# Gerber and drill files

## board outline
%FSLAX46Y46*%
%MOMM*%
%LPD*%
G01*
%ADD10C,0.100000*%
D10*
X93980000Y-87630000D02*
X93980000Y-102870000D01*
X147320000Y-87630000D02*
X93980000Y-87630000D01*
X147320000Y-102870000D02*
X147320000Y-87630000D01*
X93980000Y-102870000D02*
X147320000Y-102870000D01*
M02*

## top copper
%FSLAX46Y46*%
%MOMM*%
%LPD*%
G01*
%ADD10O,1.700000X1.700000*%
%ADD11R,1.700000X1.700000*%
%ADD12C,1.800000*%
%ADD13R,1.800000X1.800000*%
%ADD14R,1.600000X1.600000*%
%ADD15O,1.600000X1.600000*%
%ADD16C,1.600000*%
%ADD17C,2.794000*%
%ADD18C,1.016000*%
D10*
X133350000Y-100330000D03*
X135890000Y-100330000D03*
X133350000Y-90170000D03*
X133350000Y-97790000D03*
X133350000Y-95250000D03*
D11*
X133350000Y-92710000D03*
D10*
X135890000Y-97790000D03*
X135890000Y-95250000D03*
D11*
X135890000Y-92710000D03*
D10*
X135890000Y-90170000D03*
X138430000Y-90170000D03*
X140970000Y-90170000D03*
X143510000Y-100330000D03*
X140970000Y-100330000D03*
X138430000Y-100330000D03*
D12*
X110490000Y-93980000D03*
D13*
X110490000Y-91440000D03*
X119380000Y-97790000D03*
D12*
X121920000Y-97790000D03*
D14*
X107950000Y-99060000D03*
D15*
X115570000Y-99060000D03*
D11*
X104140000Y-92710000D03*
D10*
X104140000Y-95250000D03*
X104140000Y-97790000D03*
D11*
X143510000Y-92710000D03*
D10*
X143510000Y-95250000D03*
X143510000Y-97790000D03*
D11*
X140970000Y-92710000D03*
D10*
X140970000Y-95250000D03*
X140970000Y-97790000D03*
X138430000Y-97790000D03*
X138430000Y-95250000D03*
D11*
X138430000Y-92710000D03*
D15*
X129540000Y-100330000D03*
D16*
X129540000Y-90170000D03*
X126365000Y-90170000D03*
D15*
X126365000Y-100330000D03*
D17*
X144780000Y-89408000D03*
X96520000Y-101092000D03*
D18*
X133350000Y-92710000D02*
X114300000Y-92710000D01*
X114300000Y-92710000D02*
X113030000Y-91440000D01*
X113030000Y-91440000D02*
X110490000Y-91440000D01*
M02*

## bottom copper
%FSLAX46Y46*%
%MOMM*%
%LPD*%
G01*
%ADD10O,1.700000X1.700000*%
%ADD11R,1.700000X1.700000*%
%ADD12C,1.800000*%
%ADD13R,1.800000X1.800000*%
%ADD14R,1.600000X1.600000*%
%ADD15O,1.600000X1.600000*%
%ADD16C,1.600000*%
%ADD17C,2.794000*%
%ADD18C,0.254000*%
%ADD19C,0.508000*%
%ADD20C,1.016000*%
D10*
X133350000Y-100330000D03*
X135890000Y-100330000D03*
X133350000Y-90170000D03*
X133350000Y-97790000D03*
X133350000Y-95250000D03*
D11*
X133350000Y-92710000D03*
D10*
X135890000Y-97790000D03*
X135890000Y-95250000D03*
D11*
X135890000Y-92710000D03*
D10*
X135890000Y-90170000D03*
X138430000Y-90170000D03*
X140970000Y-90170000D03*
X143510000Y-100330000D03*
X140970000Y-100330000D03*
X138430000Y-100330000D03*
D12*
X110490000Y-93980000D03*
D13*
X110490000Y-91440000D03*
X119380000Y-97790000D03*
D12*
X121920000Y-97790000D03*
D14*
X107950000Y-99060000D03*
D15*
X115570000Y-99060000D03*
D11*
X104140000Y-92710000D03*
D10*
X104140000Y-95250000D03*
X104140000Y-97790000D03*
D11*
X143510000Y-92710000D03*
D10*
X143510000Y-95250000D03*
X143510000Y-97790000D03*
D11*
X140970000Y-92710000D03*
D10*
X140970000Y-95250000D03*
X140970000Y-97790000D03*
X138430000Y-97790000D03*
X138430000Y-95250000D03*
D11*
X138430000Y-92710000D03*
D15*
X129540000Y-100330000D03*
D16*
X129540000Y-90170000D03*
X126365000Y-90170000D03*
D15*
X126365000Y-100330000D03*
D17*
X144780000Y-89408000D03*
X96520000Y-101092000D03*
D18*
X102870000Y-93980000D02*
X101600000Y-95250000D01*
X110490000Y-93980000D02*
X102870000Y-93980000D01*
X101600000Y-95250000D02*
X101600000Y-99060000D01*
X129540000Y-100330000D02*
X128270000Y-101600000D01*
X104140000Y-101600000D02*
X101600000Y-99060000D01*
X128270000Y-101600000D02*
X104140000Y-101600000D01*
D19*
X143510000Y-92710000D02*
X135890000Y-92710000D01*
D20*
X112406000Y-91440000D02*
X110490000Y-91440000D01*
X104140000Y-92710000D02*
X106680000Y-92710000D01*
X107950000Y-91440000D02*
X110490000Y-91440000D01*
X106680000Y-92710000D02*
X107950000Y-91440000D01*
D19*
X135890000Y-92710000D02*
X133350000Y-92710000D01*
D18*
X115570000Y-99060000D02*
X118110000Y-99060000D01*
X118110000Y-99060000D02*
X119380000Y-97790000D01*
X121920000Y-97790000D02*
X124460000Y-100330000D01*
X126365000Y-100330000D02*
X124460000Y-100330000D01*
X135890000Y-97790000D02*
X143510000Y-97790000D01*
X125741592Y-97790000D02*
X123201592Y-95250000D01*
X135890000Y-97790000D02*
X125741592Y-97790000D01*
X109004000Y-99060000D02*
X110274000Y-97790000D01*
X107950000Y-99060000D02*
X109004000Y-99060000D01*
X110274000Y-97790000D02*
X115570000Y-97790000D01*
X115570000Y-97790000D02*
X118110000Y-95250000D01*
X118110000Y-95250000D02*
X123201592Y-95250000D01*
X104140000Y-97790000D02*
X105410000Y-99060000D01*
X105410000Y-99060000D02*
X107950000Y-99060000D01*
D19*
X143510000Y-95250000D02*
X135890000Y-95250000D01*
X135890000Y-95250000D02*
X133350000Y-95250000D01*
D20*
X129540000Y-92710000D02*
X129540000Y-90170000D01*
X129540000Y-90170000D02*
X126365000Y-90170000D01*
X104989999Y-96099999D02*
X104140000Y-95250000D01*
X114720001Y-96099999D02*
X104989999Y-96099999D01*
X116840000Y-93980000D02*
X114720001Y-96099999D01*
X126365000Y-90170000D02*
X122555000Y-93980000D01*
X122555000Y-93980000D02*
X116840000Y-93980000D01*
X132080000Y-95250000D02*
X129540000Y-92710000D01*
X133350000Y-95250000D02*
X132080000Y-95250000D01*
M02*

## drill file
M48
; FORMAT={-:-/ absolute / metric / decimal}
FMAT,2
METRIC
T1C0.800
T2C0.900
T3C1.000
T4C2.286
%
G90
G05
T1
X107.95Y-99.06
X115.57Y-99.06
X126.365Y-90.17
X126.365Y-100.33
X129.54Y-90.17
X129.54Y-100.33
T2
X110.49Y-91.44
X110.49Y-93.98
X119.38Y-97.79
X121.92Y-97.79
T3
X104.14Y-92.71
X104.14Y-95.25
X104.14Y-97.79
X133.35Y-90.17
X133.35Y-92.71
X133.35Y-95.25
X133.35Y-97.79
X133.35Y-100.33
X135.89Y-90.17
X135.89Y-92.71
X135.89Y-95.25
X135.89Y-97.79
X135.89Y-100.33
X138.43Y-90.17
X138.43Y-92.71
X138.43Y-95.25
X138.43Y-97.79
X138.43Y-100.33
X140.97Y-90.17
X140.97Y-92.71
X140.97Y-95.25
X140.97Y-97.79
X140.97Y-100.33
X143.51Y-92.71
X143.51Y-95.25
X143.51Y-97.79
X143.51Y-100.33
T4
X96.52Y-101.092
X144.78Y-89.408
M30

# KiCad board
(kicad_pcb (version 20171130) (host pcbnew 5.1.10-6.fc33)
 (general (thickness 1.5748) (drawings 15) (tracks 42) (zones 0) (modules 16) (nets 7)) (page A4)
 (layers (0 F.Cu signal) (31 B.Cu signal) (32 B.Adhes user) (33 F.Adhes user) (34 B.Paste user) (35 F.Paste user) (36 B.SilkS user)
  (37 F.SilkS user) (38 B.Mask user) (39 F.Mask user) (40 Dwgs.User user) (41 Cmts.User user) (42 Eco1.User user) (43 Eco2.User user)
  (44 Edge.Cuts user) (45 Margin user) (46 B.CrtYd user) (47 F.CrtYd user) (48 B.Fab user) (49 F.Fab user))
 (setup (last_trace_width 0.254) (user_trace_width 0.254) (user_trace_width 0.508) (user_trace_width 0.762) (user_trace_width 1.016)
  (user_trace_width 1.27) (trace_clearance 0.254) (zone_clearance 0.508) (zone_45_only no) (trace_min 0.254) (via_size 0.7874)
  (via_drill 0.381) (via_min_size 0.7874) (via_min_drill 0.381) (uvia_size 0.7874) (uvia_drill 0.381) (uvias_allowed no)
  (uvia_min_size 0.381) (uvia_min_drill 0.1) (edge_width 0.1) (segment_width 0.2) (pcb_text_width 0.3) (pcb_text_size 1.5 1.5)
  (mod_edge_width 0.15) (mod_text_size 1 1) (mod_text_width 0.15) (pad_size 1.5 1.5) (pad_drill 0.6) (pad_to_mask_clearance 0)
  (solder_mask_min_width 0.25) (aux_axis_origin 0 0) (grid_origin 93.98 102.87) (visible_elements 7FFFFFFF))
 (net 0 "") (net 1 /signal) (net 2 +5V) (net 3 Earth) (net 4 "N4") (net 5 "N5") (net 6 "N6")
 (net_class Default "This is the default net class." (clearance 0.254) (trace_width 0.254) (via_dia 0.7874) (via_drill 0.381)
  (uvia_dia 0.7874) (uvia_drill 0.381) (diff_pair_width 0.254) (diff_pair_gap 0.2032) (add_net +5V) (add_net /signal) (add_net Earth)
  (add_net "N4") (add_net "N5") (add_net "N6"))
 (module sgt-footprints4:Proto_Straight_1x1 (layer F.Cu) (at 133.35 100.33)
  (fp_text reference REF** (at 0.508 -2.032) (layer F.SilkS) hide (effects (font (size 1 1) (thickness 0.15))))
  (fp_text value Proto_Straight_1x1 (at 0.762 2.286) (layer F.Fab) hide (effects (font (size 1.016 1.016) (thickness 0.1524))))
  (pad 1 thru_hole oval (at 0 0) (size 1.7 1.7) (drill 1) (layers *.Cu *.Mask)))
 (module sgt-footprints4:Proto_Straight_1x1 (layer F.Cu) (at 135.89 100.33)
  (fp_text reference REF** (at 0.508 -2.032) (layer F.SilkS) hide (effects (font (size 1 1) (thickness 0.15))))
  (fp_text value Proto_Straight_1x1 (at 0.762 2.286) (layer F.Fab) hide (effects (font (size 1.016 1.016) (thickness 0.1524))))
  (pad 1 thru_hole oval (at 0 0) (size 1.7 1.7) (drill 1) (layers *.Cu *.Mask)))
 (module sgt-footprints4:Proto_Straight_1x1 (layer F.Cu) (at 133.35 90.17)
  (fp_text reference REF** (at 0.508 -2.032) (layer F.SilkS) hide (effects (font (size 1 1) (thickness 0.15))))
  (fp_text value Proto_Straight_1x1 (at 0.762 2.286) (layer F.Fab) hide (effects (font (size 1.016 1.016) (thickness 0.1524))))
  (pad 1 thru_hole oval (at 0 0) (size 1.7 1.7) (drill 1) (layers *.Cu *.Mask)))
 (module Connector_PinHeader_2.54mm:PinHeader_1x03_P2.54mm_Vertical (layer F.Cu) (at 133.35 92.71)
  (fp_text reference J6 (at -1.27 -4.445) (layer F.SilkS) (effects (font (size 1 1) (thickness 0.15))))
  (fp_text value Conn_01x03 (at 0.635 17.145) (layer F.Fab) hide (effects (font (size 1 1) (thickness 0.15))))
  (pad 3 thru_hole oval (at 0 5.08) (size 1.7 1.7) (drill 1) (layers *.Cu *.Mask) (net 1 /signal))
  (pad 2 thru_hole oval (at 0 2.54) (size 1.7 1.7) (drill 1) (layers *.Cu *.Mask) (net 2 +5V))
  (pad 1 thru_hole rect (at 0 0) (size 1.7 1.7) (drill 1) (layers *.Cu *.Mask) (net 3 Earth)))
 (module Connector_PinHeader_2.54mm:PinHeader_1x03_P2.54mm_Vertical (layer F.Cu) (at 135.89 92.71)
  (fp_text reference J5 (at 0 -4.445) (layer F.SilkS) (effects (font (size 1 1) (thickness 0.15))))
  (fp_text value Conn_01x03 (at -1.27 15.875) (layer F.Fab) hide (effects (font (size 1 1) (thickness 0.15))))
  (pad 3 thru_hole oval (at 0 5.08) (size 1.7 1.7) (drill 1) (layers *.Cu *.Mask) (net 1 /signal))
  (pad 2 thru_hole oval (at 0 2.54) (size 1.7 1.7) (drill 1) (layers *.Cu *.Mask) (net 2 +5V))
  (pad 1 thru_hole rect (at 0 0) (size 1.7 1.7) (drill 1) (layers *.Cu *.Mask) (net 3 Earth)))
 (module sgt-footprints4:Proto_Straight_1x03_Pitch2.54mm (layer F.Cu) (at 135.89 90.17 90)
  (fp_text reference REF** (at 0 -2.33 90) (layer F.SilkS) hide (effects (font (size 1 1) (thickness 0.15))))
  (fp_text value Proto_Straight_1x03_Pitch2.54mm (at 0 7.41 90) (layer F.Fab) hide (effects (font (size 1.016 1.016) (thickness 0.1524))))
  (pad 1 thru_hole oval (at 0 0 90) (size 1.7 1.7) (drill 1) (layers *.Cu *.Mask))
  (pad 2 thru_hole oval (at 0 2.54 90) (size 1.7 1.7) (drill 1) (layers *.Cu *.Mask))
  (pad 3 thru_hole oval (at 0 5.08 90) (size 1.7 1.7) (drill 1) (layers *.Cu *.Mask)))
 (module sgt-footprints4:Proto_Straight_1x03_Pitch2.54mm (layer F.Cu) (at 138.43 100.33 90)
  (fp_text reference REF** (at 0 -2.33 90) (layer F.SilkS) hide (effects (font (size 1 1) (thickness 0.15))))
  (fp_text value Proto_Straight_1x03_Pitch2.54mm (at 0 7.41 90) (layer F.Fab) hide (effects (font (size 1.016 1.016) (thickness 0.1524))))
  (pad 3 thru_hole oval (at 0 5.08 90) (size 1.7 1.7) (drill 1) (layers *.Cu *.Mask))
  (pad 2 thru_hole oval (at 0 2.54 90) (size 1.7 1.7) (drill 1) (layers *.Cu *.Mask))
  (pad 1 thru_hole oval (at 0 0 90) (size 1.7 1.7) (drill 1) (layers *.Cu *.Mask)))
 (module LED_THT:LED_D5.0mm (layer F.Cu) (at 110.49 91.44 270)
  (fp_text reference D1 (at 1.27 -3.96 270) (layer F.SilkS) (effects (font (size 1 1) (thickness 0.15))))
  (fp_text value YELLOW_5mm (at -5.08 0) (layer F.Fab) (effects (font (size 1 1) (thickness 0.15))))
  (pad 2 thru_hole circle (at 2.54 0 270) (size 1.8 1.8) (drill 0.9) (layers *.Cu *.Mask) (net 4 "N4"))
  (pad 1 thru_hole rect (at 0 0 270) (size 1.8 1.8) (drill 0.9) (layers *.Cu *.Mask) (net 3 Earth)))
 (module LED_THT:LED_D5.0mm (layer F.Cu) (at 119.38 97.79)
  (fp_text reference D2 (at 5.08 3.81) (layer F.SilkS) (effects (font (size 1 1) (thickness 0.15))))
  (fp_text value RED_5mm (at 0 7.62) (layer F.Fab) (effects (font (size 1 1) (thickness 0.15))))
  (pad 1 thru_hole rect (at 0 0) (size 1.8 1.8) (drill 0.9) (layers *.Cu *.Mask) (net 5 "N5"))
  (pad 2 thru_hole circle (at 2.54 0) (size 1.8 1.8) (drill 0.9) (layers *.Cu *.Mask) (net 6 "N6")))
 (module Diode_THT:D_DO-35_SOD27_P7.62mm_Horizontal (layer F.Cu) (at 107.95 99.06)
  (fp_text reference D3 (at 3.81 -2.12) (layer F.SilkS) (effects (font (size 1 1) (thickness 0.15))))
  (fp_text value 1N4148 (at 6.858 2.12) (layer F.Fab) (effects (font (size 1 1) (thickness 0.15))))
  (pad 1 thru_hole rect (at 0 0) (size 1.6 1.6) (drill 0.8) (layers *.Cu *.Mask) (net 1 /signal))
  (pad 2 thru_hole oval (at 7.62 0) (size 1.6 1.6) (drill 0.8) (layers *.Cu *.Mask) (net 5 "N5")))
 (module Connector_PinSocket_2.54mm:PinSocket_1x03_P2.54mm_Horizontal (layer F.Cu) (at 104.14 92.71)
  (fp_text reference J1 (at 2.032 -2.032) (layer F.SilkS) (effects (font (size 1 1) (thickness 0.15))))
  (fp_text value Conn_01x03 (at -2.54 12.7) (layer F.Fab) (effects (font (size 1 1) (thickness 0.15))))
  (pad 1 thru_hole rect (at 0 0) (size 1.7 1.7) (drill 1) (layers *.Cu *.Mask) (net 3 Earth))
  (pad 2 thru_hole oval (at 0 2.54) (size 1.7 1.7) (drill 1) (layers *.Cu *.Mask) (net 2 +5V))
  (pad 3 thru_hole oval (at 0 5.08) (size 1.7 1.7) (drill 1) (layers *.Cu *.Mask) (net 1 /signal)))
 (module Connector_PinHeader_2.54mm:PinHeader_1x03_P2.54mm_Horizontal (layer F.Cu) (at 143.51 92.71)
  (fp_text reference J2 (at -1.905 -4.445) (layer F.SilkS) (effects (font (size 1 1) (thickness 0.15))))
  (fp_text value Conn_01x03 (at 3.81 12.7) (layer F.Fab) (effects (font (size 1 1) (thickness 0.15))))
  (pad 1 thru_hole rect (at 0 0) (size 1.7 1.7) (drill 1) (layers *.Cu *.Mask) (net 3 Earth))
  (pad 2 thru_hole oval (at 0 2.54) (size 1.7 1.7) (drill 1) (layers *.Cu *.Mask) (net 2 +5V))
  (pad 3 thru_hole oval (at 0 5.08) (size 1.7 1.7) (drill 1) (layers *.Cu *.Mask) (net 1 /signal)))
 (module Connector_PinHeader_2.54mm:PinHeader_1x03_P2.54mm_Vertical (layer F.Cu) (at 140.97 92.71)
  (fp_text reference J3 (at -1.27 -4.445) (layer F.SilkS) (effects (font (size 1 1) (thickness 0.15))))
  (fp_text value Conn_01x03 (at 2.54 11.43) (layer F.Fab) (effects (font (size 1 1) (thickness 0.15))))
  (pad 1 thru_hole rect (at 0 0) (size 1.7 1.7) (drill 1) (layers *.Cu *.Mask) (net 3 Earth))
  (pad 2 thru_hole oval (at 0 2.54) (size 1.7 1.7) (drill 1) (layers *.Cu *.Mask) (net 2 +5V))
  (pad 3 thru_hole oval (at 0 5.08) (size 1.7 1.7) (drill 1) (layers *.Cu *.Mask) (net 1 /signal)))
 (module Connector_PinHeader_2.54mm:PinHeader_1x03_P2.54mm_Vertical (layer F.Cu) (at 138.43 92.71)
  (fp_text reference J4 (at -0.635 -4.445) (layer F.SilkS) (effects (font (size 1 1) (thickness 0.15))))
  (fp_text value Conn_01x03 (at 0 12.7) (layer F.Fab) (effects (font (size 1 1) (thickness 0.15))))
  (pad 3 thru_hole oval (at 0 5.08) (size 1.7 1.7) (drill 1) (layers *.Cu *.Mask) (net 1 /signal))
  (pad 2 thru_hole oval (at 0 2.54) (size 1.7 1.7) (drill 1) (layers *.Cu *.Mask) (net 2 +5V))
  (pad 1 thru_hole rect (at 0 0) (size 1.7 1.7) (drill 1) (layers *.Cu *.Mask) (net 3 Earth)))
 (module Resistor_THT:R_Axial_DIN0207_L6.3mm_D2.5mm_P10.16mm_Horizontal (layer F.Cu) (at 129.54 90.17 270)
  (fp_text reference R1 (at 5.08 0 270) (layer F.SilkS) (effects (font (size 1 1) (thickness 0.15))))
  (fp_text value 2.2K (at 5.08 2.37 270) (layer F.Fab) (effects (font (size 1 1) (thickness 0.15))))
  (pad 2 thru_hole oval (at 10.16 0 270) (size 1.6 1.6) (drill 0.8) (layers *.Cu *.Mask) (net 4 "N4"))
  (pad 1 thru_hole circle (at 0 0 270) (size 1.6 1.6) (drill 0.8) (layers *.Cu *.Mask) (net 2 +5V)))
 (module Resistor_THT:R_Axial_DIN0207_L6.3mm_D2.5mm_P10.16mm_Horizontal (layer F.Cu) (at 126.365 90.17 270)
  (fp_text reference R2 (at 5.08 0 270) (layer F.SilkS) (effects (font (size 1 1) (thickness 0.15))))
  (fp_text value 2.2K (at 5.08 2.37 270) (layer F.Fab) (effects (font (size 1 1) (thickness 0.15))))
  (pad 1 thru_hole circle (at 0 0 270) (size 1.6 1.6) (drill 0.8) (layers *.Cu *.Mask) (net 2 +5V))
  (pad 2 thru_hole oval (at 10.16 0 270) (size 1.6 1.6) (drill 0.8) (layers *.Cu *.Mask) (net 6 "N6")))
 (gr_line (start 93.98 87.63) (end 93.98 102.87) (layer Edge.Cuts) (width 0.1))
 (gr_line (start 147.32 87.63) (end 93.98 87.63) (layer Edge.Cuts) (width 0.1))
 (gr_line (start 147.32 102.87) (end 147.32 87.63) (layer Edge.Cuts) (width 0.1))
 (gr_line (start 93.98 102.87) (end 147.32 102.87) (layer Edge.Cuts) (width 0.1))
 (via (at 144.78 89.408) (size 2.794) (drill 2.286) (layers F.Cu B.Cu) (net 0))
 (via (at 96.52 101.092) (size 2.794) (drill 2.286) (layers F.Cu B.Cu) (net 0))
 (segment (start 102.87 93.98) (end 101.6 95.25) (width 0.254) (layer B.Cu) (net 4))
 (segment (start 110.49 93.98) (end 102.87 93.98) (width 0.254) (layer B.Cu) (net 4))
 (segment (start 101.6 95.25) (end 101.6 99.06) (width 0.254) (layer B.Cu) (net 4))
 (segment (start 129.54 100.33) (end 128.27 101.6) (width 0.254) (layer B.Cu) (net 4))
 (segment (start 104.14 101.6) (end 101.6 99.06) (width 0.254) (layer B.Cu) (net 4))
 (segment (start 128.27 101.6) (end 104.14 101.6) (width 0.254) (layer B.Cu) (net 4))
 (segment (start 143.51 92.71) (end 135.89 92.71) (width 0.508) (layer B.Cu) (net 3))
 (segment (start 112.406 91.44) (end 110.49 91.44) (width 1.016) (layer B.Cu) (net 3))
 (segment (start 104.14 92.71) (end 106.68 92.71) (width 1.016) (layer B.Cu) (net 3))
 (segment (start 107.95 91.44) (end 110.49 91.44) (width 1.016) (layer B.Cu) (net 3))
 (segment (start 106.68 92.71) (end 107.95 91.44) (width 1.016) (layer B.Cu) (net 3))
 (segment (start 135.89 92.71) (end 133.35 92.71) (width 0.508) (layer B.Cu) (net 3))
 (segment (start 133.35 92.71) (end 114.3 92.71) (width 1.016) (layer F.Cu) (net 3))
 (segment (start 114.3 92.71) (end 113.03 91.44) (width 1.016) (layer F.Cu) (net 3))
 (segment (start 113.03 91.44) (end 110.49 91.44) (width 1.016) (layer F.Cu) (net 3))
 (segment (start 115.57 99.06) (end 118.11 99.06) (width 0.254) (layer B.Cu) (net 5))
 (segment (start 118.11 99.06) (end 119.38 97.79) (width 0.254) (layer B.Cu) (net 5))
 (segment (start 121.92 97.79) (end 124.46 100.33) (width 0.254) (layer B.Cu) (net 6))
 (segment (start 126.365 100.33) (end 124.46 100.33) (width 0.254) (layer B.Cu) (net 6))
 (segment (start 135.89 97.79) (end 143.51 97.79) (width 0.254) (layer B.Cu) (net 1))
 (segment (start 125.741592 97.79) (end 123.201592 95.25) (width 0.254) (layer B.Cu) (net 1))
 (segment (start 135.89 97.79) (end 125.741592 97.79) (width 0.254) (layer B.Cu) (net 1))
 (segment (start 109.004 99.06) (end 110.274 97.79) (width 0.254) (layer B.Cu) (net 1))
 (segment (start 107.95 99.06) (end 109.004 99.06) (width 0.254) (layer B.Cu) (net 1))
 (segment (start 110.274 97.79) (end 115.57 97.79) (width 0.254) (layer B.Cu) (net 1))
 (segment (start 115.57 97.79) (end 118.11 95.25) (width 0.254) (layer B.Cu) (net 1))
 (segment (start 118.11 95.25) (end 123.201592 95.25) (width 0.254) (layer B.Cu) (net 1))
 (segment (start 104.14 97.79) (end 105.41 99.06) (width 0.254) (layer B.Cu) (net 1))
 (segment (start 105.41 99.06) (end 107.95 99.06) (width 0.254) (layer B.Cu) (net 1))
 (segment (start 143.51 95.25) (end 135.89 95.25) (width 0.508) (layer B.Cu) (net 2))
 (segment (start 135.89 95.25) (end 133.35 95.25) (width 0.508) (layer B.Cu) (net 2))
 (segment (start 129.54 92.71) (end 129.54 90.17) (width 1.016) (layer B.Cu) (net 2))
 (segment (start 129.54 90.17) (end 126.365 90.17) (width 1.016) (layer B.Cu) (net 2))
 (segment (start 104.989999 96.099999) (end 104.14 95.25) (width 1.016) (layer B.Cu) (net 2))
 (segment (start 114.720001 96.099999) (end 104.989999 96.099999) (width 1.016) (layer B.Cu) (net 2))
 (segment (start 116.84 93.98) (end 114.720001 96.099999) (width 1.016) (layer B.Cu) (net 2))
 (segment (start 126.365 90.17) (end 122.555 93.98) (width 1.016) (layer B.Cu) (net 2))
 (segment (start 122.555 93.98) (end 116.84 93.98) (width 1.016) (layer B.Cu) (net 2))
 (segment (start 132.08 95.25) (end 129.54 92.71) (width 1.016) (layer B.Cu) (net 2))
 (segment (start 133.35 95.25) (end 132.08 95.25) (width 1.016) (layer B.Cu) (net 2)))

